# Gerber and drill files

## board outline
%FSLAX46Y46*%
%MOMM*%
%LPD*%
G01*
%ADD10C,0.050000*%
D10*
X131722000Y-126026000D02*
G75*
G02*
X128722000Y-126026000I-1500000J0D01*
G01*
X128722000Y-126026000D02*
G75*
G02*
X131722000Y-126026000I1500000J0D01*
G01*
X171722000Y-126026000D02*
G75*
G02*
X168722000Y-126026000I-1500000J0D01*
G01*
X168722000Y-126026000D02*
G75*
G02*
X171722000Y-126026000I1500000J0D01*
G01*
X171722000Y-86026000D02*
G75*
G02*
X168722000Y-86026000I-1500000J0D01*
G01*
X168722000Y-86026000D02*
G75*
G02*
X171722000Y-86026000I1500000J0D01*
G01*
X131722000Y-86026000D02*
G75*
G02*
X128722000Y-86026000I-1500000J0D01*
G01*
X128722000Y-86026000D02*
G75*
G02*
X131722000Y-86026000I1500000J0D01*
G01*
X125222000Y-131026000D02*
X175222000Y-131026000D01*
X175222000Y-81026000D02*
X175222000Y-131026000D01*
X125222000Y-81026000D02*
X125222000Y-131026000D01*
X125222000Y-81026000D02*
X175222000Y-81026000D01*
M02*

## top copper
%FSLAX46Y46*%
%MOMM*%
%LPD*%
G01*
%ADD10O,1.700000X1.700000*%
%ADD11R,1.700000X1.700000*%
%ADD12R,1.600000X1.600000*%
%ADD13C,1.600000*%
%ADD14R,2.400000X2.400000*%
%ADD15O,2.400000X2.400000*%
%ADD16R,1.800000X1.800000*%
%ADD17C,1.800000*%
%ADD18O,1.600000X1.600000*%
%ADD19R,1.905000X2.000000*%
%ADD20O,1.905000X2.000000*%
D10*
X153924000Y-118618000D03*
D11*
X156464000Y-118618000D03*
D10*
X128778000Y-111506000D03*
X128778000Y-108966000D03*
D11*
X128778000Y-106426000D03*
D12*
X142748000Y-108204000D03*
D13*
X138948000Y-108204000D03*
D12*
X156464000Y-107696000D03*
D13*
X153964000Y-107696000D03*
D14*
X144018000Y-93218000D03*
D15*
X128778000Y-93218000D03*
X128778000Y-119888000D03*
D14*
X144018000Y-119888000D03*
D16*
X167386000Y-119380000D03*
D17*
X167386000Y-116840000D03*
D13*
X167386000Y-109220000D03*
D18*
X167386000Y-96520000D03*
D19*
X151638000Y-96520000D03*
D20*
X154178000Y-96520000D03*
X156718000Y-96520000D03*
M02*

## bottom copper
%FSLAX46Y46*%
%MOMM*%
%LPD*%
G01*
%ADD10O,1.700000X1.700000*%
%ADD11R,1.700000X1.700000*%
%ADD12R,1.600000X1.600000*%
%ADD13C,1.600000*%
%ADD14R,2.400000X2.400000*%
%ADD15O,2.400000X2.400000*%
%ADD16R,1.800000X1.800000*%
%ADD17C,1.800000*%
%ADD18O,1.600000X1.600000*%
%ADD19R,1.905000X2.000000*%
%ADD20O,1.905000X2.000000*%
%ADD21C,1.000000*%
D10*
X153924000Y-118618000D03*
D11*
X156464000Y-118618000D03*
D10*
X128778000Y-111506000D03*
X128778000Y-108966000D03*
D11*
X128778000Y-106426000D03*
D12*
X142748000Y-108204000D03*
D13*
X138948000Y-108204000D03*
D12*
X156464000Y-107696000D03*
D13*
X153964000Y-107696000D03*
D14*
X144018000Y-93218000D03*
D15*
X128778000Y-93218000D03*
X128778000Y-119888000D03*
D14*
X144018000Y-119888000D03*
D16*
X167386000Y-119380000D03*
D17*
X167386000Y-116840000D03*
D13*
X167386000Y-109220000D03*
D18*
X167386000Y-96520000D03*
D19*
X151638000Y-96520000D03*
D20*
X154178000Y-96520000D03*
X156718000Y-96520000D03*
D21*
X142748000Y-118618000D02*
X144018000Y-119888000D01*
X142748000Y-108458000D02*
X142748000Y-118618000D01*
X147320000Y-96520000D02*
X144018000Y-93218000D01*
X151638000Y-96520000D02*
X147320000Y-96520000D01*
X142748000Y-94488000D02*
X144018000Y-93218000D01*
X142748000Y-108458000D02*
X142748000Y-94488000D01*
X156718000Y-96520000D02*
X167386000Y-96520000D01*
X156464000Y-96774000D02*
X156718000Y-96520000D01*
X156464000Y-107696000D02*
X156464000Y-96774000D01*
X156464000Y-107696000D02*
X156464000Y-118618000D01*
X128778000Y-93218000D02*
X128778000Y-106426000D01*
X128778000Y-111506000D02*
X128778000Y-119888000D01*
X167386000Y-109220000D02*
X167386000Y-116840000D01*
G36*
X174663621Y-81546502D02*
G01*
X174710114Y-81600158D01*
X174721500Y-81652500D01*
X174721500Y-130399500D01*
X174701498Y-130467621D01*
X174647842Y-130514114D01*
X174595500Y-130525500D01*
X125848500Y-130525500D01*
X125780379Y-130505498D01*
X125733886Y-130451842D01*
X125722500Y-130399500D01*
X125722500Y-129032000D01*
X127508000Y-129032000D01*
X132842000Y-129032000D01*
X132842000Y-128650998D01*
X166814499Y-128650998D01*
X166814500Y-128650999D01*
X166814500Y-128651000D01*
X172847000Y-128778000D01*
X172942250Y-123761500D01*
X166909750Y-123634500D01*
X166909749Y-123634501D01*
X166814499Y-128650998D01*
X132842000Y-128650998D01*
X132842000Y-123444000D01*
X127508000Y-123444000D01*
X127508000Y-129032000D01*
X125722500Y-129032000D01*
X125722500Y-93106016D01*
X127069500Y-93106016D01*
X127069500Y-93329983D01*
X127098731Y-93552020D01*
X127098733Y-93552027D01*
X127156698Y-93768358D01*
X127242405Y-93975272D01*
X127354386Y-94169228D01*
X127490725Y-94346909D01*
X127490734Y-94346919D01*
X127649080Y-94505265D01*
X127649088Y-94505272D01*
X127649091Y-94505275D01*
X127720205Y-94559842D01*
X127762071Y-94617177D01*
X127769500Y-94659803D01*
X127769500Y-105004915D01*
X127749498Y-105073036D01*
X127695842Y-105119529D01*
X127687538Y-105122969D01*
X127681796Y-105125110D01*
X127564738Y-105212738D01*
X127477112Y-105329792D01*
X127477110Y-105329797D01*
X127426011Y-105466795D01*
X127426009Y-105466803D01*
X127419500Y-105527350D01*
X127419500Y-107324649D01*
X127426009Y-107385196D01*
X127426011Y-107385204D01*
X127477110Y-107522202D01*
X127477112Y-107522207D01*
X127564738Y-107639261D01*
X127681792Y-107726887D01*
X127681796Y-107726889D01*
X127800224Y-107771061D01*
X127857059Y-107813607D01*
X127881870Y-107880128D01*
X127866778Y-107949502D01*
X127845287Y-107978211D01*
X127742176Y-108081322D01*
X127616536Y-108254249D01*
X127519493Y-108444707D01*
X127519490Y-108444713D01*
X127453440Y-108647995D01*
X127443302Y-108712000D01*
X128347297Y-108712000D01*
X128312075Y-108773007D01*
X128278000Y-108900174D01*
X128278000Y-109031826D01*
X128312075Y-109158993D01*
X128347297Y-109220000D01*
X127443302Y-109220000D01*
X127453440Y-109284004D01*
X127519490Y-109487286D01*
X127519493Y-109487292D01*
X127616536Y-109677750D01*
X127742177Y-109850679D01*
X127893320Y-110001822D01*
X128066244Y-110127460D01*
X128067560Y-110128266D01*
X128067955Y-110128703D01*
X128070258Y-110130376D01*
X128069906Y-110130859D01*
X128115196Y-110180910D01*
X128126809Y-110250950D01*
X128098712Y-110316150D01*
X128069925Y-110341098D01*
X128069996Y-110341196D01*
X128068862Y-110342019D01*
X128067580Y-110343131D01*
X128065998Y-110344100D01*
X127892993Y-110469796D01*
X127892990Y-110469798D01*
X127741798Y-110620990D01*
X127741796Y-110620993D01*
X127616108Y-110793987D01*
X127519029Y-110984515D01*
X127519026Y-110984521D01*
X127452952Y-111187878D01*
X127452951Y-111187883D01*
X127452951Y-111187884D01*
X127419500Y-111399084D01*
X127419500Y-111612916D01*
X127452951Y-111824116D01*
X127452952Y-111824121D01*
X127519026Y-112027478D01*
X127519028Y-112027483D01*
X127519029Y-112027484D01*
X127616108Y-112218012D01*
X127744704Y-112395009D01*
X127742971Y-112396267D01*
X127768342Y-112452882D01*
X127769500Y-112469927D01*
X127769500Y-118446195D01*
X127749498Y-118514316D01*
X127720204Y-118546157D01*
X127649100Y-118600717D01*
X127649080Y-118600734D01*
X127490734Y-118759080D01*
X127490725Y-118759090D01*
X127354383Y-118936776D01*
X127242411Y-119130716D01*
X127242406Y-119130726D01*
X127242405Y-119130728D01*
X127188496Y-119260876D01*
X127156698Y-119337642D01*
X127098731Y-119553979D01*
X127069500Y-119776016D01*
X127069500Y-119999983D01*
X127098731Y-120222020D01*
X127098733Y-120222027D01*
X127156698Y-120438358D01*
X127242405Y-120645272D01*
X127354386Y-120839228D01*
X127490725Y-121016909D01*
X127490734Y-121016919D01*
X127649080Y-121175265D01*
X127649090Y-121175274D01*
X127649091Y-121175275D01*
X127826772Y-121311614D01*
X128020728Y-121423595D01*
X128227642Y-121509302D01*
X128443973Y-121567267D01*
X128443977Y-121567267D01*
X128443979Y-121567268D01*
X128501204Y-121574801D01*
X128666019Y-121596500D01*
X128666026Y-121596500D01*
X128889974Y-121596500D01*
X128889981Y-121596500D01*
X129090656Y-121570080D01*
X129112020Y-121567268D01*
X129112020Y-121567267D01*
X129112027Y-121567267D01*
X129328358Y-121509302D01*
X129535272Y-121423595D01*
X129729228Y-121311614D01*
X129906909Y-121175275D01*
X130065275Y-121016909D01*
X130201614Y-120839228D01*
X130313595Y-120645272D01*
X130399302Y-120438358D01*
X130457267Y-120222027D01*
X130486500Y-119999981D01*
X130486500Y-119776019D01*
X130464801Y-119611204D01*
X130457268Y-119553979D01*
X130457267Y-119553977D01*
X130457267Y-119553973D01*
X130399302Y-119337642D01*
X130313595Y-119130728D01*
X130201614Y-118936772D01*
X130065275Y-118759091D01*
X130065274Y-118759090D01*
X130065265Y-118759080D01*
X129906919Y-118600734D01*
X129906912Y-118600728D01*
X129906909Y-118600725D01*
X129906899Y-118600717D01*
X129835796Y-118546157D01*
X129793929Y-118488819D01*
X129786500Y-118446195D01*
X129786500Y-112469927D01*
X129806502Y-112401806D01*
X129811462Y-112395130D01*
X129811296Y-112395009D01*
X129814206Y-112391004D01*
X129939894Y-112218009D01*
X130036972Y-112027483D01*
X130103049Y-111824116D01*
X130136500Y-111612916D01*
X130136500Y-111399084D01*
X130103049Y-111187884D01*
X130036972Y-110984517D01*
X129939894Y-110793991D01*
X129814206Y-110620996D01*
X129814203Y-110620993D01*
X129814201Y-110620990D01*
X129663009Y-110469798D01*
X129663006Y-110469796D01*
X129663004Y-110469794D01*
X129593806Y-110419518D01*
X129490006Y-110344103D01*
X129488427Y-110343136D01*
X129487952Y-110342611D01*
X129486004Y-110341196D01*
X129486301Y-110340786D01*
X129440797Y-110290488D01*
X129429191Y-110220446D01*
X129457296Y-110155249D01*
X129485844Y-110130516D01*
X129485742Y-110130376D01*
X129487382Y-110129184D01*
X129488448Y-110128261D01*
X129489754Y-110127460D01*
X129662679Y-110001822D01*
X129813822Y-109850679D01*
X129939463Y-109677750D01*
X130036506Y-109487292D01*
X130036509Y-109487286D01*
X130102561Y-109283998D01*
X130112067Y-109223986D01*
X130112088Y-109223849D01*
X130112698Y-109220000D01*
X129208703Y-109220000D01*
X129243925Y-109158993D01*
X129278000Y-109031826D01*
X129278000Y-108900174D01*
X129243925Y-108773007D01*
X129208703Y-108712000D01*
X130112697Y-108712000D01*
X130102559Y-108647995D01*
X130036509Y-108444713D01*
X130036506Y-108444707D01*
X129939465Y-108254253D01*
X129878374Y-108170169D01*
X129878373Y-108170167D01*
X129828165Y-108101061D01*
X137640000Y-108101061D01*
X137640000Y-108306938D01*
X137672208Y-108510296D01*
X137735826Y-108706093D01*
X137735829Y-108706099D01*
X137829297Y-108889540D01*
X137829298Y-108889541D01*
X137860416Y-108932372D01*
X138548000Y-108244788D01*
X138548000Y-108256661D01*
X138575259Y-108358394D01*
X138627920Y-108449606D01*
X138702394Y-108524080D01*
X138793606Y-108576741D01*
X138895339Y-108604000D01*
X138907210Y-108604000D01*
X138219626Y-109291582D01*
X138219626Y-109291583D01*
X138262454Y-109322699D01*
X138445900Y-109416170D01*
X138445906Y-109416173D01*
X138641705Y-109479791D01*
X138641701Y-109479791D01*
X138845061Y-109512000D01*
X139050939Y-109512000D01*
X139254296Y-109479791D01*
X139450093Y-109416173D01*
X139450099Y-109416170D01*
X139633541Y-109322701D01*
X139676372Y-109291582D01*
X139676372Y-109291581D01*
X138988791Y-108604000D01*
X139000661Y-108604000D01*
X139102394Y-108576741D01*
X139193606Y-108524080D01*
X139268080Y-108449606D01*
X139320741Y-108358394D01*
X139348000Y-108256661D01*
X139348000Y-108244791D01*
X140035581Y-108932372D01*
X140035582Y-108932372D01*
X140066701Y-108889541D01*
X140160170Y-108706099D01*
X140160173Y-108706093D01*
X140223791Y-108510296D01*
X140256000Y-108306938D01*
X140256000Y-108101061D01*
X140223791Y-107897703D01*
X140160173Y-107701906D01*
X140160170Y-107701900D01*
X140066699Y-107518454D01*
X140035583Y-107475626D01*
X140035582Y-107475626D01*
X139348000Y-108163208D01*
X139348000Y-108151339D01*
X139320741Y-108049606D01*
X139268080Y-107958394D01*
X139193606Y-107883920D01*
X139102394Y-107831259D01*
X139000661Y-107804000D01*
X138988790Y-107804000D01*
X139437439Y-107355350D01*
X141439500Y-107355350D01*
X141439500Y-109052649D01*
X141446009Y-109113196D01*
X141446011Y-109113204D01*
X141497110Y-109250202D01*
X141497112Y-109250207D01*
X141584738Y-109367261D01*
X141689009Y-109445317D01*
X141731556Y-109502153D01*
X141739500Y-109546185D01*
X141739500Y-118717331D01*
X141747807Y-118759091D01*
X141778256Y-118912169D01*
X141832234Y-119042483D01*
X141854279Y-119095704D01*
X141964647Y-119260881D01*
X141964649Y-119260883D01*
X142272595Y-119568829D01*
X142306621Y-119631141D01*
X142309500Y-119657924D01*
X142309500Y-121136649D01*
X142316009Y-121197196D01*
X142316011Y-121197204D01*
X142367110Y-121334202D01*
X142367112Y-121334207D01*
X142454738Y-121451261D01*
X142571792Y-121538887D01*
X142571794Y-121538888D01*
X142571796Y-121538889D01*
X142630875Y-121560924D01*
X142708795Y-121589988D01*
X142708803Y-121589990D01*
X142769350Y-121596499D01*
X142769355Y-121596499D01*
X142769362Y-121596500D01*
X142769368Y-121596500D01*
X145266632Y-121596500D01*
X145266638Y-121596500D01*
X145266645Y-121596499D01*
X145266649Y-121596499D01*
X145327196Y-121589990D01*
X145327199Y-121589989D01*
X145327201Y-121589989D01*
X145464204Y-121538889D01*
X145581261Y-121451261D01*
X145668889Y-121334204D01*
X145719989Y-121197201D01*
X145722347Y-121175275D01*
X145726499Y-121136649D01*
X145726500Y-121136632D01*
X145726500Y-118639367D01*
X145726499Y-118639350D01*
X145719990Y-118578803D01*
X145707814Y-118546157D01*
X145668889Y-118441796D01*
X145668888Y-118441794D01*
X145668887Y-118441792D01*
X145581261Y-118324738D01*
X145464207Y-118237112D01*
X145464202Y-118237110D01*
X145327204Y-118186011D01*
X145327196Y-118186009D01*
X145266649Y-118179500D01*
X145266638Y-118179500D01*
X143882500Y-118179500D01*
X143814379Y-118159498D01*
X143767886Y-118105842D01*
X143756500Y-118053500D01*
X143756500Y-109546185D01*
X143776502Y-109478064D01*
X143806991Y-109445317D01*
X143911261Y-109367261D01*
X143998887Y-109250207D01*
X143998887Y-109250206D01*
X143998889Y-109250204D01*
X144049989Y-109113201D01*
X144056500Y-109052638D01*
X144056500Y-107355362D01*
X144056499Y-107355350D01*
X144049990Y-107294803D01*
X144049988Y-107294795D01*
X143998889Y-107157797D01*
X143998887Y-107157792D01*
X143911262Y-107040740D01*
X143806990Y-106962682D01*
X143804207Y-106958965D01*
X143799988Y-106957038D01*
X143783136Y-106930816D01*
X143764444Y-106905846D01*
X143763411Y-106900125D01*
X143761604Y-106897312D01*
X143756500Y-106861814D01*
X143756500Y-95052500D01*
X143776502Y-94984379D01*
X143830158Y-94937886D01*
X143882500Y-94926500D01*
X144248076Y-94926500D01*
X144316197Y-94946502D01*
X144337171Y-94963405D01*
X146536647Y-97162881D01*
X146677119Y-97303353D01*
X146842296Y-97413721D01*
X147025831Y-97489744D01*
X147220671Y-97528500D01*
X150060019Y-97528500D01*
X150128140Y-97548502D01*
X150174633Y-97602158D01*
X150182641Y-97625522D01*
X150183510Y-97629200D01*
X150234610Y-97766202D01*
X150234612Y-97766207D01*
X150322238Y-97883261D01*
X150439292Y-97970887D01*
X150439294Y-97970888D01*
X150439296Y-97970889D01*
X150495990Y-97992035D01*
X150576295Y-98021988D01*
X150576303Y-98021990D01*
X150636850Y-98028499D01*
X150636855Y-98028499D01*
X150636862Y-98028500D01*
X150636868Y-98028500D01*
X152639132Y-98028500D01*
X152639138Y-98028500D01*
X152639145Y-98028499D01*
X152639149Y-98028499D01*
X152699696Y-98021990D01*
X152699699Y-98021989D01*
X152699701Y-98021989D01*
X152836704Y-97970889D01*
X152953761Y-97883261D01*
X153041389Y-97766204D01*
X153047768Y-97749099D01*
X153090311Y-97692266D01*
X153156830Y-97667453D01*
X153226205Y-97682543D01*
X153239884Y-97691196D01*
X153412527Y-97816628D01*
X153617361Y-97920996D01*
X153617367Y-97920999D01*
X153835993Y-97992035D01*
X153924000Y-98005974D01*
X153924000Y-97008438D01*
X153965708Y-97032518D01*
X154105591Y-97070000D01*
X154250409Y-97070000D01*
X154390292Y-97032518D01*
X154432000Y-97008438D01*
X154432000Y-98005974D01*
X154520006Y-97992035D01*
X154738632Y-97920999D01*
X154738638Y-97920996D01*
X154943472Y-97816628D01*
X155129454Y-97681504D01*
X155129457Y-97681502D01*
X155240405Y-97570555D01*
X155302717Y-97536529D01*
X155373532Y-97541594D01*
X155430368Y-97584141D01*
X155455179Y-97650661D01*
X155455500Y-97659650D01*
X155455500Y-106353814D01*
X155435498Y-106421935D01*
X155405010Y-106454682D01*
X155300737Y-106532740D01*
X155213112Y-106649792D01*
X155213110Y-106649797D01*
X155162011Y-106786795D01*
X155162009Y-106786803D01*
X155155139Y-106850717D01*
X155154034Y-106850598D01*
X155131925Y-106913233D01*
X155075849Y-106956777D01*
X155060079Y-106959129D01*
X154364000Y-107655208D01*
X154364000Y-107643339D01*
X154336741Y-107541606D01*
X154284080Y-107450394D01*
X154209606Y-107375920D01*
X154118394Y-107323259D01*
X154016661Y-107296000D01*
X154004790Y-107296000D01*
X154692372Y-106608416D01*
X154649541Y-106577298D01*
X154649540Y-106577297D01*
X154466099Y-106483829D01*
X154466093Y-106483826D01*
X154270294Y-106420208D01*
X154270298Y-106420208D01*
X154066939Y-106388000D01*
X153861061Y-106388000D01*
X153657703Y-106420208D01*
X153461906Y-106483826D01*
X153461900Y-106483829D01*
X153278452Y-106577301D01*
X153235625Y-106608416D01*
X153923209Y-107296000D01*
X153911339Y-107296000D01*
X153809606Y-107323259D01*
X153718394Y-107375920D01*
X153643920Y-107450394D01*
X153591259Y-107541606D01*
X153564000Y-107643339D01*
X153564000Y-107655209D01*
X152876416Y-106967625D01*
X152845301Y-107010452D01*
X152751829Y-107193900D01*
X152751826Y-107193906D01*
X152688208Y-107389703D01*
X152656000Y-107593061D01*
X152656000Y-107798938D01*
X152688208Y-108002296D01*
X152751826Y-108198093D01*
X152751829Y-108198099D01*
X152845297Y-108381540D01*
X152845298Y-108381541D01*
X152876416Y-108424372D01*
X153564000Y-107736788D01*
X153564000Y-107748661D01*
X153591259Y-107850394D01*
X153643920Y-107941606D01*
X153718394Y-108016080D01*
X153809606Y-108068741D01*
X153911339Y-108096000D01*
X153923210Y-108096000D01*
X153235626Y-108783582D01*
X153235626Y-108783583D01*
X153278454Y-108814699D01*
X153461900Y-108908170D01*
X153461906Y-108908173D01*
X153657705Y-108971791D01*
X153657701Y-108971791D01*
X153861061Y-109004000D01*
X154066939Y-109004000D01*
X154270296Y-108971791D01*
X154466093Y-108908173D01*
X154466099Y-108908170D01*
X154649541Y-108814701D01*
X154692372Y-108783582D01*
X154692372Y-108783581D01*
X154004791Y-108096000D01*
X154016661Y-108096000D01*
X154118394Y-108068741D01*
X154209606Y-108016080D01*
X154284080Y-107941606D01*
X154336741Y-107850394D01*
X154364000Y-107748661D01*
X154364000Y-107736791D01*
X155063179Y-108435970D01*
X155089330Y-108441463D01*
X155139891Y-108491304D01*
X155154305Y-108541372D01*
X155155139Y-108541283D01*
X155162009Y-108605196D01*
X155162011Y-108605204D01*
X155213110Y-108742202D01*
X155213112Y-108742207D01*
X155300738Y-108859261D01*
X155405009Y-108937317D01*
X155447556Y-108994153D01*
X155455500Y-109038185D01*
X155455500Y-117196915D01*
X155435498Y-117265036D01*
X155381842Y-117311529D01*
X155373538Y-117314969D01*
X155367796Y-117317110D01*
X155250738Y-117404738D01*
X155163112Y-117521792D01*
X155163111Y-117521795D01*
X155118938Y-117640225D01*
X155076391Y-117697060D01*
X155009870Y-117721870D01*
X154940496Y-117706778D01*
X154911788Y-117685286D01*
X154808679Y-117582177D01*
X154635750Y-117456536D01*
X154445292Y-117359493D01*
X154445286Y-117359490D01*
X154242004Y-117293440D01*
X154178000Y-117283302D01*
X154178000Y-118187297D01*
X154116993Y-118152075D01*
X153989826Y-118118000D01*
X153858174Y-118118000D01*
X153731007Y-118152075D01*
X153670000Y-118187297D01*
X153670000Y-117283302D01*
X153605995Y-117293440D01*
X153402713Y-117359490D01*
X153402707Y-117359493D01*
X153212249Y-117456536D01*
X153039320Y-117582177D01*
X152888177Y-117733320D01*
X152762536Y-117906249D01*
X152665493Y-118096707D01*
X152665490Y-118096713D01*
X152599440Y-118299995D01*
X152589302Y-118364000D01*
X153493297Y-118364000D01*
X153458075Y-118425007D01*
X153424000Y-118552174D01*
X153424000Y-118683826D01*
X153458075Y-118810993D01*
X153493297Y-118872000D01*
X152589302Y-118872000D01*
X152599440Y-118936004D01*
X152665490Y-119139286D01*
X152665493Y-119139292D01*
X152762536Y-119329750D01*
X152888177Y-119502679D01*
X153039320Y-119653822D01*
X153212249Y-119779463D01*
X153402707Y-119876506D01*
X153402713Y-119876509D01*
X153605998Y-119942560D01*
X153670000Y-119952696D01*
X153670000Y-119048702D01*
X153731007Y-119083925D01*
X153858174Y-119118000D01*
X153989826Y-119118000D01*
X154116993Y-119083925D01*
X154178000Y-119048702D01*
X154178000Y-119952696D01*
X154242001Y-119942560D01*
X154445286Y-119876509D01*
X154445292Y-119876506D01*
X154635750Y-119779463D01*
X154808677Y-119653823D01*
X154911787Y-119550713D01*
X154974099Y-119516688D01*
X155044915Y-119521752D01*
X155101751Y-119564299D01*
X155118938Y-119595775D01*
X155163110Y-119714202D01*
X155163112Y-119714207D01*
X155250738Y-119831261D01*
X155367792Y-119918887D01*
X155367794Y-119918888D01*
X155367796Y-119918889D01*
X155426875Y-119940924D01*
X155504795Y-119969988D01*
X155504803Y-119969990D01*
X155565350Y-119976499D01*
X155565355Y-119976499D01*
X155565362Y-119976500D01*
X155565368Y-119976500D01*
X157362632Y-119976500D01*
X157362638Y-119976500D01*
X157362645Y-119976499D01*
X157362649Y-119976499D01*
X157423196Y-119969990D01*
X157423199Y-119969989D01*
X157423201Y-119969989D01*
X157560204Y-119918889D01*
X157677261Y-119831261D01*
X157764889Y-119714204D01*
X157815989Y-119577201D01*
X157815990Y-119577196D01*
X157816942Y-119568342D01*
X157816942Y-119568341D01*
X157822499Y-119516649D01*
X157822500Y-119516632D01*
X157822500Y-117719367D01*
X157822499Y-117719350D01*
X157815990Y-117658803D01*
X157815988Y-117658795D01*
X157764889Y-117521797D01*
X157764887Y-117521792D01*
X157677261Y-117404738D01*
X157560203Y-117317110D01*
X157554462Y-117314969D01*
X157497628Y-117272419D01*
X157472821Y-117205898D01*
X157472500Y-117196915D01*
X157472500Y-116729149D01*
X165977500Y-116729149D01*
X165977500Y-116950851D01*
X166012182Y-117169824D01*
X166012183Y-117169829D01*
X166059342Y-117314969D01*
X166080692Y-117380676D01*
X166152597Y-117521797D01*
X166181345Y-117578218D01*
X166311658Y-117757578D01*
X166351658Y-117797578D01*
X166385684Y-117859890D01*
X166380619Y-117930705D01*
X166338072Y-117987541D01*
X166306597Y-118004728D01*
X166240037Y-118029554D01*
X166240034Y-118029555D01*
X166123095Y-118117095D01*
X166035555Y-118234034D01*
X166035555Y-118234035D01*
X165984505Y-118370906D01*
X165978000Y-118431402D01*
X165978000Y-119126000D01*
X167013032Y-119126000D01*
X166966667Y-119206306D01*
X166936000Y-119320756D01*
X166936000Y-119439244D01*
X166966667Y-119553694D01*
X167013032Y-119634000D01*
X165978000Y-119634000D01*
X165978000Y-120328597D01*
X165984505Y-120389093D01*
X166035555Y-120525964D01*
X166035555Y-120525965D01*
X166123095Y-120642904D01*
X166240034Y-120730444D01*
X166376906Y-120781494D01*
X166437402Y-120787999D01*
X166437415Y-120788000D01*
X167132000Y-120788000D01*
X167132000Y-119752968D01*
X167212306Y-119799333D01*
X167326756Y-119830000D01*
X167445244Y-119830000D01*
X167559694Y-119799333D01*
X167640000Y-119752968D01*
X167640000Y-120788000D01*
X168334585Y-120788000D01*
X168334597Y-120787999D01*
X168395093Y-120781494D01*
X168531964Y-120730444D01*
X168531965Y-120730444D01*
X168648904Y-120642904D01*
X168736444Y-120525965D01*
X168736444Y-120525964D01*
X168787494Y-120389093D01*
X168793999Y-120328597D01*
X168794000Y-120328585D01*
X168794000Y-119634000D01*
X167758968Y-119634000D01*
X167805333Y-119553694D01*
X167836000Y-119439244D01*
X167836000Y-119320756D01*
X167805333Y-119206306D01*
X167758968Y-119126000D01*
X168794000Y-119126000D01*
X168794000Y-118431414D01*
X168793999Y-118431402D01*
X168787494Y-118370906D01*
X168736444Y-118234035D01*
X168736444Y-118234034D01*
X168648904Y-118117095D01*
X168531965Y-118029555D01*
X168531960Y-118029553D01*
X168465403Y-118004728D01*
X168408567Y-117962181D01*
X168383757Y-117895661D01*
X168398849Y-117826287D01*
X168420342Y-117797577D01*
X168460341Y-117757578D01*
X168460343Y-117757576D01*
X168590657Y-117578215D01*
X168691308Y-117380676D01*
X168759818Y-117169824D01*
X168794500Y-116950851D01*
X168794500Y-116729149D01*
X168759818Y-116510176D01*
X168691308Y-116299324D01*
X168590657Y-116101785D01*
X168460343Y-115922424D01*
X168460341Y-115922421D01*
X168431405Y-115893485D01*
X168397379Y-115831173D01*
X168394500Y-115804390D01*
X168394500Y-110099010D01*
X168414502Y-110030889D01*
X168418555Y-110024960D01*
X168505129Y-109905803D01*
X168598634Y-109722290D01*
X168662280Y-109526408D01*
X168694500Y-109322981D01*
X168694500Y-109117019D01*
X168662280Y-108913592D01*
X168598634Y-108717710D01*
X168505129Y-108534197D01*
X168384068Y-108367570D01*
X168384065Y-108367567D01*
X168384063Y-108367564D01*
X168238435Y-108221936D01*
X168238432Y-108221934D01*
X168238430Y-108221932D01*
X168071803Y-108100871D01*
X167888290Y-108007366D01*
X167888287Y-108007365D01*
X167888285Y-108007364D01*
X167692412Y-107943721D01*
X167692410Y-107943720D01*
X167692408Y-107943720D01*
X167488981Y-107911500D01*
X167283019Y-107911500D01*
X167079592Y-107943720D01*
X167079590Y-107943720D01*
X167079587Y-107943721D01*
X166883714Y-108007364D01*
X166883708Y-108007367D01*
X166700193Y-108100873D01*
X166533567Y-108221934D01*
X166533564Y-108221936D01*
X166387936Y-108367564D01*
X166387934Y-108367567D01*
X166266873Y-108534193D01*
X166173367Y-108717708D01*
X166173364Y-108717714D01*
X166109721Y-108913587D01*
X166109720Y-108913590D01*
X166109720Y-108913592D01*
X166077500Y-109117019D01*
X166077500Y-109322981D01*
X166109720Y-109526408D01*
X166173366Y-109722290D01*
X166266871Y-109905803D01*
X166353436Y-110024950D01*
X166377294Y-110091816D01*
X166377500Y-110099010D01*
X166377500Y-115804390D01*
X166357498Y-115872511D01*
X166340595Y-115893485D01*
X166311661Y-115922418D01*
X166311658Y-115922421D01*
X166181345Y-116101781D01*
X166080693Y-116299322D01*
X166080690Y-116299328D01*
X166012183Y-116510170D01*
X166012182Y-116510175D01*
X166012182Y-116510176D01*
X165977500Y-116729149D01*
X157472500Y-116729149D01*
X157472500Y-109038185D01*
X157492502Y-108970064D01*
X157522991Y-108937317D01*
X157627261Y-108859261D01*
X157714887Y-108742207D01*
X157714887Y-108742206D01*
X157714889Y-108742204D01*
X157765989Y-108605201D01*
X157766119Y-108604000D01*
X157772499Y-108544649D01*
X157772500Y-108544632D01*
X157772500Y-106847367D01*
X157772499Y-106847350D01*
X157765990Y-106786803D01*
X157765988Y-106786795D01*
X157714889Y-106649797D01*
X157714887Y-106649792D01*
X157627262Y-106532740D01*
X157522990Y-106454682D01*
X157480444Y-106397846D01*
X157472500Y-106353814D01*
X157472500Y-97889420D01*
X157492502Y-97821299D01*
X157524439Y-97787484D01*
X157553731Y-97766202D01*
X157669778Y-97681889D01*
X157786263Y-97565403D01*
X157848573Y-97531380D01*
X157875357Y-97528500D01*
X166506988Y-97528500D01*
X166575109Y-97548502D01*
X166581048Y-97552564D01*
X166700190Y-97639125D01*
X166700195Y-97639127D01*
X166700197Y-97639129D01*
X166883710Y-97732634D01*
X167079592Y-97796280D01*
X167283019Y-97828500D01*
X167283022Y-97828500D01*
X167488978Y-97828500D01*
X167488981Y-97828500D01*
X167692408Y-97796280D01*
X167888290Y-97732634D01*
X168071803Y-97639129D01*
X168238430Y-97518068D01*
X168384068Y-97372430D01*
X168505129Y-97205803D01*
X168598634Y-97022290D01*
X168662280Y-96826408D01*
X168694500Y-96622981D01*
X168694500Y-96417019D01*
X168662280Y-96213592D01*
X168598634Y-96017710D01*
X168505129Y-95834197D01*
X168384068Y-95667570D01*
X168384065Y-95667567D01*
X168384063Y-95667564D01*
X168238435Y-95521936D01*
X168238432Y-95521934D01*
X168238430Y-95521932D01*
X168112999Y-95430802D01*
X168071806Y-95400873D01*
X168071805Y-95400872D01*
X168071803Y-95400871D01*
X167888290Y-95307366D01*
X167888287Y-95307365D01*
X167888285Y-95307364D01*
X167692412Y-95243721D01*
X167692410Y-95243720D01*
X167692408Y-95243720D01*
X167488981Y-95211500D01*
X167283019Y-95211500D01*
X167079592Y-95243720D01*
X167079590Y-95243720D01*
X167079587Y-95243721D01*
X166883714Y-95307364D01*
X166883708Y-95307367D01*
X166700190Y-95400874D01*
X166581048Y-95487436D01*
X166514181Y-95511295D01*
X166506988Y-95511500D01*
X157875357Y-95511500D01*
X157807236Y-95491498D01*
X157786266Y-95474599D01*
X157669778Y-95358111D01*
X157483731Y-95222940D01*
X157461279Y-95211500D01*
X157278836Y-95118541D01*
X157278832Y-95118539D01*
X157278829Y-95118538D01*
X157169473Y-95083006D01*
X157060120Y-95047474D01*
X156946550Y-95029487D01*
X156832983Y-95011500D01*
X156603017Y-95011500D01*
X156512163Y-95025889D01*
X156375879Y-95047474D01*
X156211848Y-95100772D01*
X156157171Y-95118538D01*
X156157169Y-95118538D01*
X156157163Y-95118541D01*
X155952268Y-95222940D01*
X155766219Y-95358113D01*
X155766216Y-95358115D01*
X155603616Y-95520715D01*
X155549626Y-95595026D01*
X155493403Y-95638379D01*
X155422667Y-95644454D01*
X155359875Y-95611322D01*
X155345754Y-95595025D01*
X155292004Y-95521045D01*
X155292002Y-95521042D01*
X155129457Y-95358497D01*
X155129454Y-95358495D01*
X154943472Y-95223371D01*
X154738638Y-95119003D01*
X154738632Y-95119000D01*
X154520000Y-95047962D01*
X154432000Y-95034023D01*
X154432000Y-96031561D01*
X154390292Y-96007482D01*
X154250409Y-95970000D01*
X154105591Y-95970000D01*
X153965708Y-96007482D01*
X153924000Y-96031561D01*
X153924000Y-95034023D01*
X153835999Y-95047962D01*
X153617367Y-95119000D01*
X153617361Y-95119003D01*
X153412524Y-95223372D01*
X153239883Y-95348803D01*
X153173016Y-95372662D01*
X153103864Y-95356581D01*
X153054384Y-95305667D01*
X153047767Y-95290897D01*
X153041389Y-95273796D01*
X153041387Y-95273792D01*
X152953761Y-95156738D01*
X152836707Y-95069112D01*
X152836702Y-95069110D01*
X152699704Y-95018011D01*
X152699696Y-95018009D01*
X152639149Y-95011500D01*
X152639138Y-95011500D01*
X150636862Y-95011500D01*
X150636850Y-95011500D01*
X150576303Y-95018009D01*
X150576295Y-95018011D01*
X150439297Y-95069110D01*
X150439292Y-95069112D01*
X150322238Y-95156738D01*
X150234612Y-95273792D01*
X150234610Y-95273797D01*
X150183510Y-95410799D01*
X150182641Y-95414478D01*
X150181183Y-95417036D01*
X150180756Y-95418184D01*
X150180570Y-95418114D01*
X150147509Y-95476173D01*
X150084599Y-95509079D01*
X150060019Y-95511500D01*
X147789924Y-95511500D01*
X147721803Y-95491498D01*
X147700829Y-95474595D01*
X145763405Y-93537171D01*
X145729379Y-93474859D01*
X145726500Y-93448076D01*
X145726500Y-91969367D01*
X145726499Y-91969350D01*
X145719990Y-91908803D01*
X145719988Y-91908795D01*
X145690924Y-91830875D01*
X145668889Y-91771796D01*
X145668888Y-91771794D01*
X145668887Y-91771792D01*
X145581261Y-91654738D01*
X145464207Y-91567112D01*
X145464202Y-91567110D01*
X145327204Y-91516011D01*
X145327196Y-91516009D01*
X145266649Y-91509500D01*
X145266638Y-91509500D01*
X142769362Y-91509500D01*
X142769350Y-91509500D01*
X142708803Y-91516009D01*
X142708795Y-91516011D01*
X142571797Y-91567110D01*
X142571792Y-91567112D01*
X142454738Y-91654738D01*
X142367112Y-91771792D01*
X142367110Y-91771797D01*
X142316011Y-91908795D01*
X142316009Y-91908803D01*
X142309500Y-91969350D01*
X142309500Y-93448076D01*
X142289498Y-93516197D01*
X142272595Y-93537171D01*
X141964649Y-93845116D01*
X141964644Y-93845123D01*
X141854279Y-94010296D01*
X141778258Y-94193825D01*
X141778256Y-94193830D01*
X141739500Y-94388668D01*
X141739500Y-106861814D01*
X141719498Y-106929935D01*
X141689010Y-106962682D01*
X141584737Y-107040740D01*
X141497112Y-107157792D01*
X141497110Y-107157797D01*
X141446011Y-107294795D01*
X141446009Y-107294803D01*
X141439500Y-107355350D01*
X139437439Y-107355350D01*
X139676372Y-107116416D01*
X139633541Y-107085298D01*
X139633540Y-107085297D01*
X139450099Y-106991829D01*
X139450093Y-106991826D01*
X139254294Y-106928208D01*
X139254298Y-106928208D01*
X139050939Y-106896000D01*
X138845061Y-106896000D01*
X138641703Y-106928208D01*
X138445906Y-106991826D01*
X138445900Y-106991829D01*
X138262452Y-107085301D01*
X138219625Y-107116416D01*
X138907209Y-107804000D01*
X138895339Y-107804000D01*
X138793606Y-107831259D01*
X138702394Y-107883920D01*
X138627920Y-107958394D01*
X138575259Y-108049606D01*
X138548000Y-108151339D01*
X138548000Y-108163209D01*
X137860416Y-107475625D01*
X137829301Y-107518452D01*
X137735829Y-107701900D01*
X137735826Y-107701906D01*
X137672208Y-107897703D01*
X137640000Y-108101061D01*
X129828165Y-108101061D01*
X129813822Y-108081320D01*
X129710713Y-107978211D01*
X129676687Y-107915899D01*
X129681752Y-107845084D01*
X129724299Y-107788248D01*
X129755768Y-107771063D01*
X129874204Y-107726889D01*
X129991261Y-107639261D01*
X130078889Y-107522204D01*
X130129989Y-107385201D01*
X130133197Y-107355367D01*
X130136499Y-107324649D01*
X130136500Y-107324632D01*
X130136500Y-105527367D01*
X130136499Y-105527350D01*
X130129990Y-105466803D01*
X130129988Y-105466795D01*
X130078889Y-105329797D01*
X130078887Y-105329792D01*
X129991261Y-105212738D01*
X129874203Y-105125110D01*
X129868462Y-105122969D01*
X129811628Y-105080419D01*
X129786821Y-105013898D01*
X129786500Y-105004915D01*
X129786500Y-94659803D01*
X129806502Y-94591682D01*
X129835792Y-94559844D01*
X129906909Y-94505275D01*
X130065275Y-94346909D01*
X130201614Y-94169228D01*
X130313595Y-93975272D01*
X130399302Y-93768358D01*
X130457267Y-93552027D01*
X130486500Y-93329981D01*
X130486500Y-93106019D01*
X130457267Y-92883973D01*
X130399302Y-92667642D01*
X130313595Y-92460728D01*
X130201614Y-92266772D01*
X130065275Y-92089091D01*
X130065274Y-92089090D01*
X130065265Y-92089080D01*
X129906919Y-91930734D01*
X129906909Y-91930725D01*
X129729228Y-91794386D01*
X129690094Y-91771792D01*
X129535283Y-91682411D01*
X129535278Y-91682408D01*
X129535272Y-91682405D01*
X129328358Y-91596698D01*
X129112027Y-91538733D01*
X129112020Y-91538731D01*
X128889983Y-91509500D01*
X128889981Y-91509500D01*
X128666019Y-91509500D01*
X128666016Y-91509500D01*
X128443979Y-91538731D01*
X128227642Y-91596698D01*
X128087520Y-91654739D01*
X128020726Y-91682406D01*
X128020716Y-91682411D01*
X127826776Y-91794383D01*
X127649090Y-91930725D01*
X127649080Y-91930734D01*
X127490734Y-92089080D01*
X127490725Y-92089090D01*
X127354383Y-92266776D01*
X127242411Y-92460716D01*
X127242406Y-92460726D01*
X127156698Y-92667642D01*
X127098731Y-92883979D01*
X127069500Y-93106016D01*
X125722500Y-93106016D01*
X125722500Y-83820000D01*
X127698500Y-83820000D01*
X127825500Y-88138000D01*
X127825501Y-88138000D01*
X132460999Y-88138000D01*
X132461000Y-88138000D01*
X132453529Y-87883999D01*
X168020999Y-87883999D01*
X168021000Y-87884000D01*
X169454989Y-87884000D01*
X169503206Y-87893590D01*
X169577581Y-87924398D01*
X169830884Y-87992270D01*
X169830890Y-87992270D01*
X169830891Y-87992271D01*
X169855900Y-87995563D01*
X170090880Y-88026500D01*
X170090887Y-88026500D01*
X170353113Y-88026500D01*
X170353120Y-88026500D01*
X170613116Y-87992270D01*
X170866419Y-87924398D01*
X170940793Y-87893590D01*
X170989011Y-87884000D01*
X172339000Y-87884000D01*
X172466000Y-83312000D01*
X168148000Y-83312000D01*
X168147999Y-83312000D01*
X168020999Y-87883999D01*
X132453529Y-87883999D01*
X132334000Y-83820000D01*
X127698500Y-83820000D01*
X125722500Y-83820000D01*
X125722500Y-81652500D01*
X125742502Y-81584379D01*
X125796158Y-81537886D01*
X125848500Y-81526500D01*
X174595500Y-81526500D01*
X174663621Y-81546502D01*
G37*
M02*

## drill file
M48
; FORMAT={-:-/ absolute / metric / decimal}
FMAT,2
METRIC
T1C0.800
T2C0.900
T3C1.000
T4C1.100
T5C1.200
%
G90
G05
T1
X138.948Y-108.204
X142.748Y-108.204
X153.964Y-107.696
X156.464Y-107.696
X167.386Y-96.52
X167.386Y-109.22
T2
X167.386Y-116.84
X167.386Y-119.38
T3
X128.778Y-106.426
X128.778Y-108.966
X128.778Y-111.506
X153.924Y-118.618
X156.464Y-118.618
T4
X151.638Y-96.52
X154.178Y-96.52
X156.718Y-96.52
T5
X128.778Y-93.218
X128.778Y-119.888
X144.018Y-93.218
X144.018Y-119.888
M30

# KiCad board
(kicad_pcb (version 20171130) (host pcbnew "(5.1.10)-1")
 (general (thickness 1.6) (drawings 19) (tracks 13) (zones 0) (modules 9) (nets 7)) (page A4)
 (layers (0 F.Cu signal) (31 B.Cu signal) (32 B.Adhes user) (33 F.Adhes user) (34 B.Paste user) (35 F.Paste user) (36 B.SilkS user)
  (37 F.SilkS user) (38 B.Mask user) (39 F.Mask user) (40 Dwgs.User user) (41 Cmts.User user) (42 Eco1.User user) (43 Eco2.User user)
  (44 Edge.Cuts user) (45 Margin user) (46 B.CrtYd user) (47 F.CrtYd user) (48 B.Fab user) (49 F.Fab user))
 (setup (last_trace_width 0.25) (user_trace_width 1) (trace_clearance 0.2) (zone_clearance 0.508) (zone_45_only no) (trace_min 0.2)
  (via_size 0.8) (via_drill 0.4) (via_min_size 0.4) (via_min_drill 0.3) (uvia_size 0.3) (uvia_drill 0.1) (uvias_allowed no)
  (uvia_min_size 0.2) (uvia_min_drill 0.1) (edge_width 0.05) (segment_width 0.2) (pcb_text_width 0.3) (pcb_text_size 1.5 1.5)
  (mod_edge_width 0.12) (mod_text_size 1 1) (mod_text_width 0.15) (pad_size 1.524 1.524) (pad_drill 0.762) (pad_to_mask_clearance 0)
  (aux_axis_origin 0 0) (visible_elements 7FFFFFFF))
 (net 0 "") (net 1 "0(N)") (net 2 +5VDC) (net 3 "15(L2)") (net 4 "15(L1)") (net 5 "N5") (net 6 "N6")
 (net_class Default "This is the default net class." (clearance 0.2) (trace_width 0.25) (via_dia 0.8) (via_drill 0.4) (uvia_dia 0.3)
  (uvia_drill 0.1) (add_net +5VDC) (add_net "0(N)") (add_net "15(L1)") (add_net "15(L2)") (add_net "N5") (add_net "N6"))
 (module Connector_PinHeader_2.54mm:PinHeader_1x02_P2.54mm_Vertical (layer F.Cu) (at 156.464 118.618 270)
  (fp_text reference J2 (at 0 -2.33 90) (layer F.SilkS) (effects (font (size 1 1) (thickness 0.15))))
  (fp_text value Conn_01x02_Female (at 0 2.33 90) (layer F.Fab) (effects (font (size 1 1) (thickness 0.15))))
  (pad 2 thru_hole oval (at 0 2.54 270) (size 1.7 1.7) (drill 1) (layers *.Cu *.Mask) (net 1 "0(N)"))
  (pad 1 thru_hole rect (at 0 0 270) (size 1.7 1.7) (drill 1) (layers *.Cu *.Mask) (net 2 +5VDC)))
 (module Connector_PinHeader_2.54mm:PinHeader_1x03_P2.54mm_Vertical (layer F.Cu) (at 128.778 106.426)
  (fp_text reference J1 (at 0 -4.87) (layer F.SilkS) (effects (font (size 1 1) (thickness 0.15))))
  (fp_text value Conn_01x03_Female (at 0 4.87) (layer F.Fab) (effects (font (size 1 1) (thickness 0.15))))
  (pad 3 thru_hole oval (at 0 5.08) (size 1.7 1.7) (drill 1) (layers *.Cu *.Mask) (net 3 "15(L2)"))
  (pad 2 thru_hole oval (at 0 2.54) (size 1.7 1.7) (drill 1) (layers *.Cu *.Mask) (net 1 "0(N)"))
  (pad 1 thru_hole rect (at 0 0) (size 1.7 1.7) (drill 1) (layers *.Cu *.Mask) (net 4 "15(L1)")))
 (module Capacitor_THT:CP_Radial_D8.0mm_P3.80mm (layer F.Cu) (at 142.748 108.204 180)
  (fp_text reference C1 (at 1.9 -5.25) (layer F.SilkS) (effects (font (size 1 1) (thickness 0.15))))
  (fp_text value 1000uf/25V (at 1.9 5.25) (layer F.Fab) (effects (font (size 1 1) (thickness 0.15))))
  (pad 1 thru_hole rect (at 0 0 180) (size 1.6 1.6) (drill 0.8) (layers *.Cu *.Mask) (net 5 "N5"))
  (pad 2 thru_hole circle (at 3.8 0 180) (size 1.6 1.6) (drill 0.8) (layers *.Cu *.Mask) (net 1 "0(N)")))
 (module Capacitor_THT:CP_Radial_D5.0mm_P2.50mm (layer F.Cu) (at 156.464 107.696 180)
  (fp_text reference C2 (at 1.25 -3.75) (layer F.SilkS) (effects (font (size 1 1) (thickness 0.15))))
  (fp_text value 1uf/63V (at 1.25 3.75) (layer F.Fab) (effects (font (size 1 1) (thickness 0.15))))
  (pad 1 thru_hole rect (at 0 0 180) (size 1.6 1.6) (drill 0.8) (layers *.Cu *.Mask) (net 2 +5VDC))
  (pad 2 thru_hole circle (at 2.5 0 180) (size 1.6 1.6) (drill 0.8) (layers *.Cu *.Mask) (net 1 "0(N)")))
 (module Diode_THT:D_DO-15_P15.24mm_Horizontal (layer F.Cu) (at 144.018 93.218 180)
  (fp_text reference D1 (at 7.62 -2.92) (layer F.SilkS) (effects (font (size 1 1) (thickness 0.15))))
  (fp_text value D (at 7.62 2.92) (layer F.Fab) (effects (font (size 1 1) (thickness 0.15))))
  (pad 1 thru_hole rect (at 0 0 180) (size 2.4 2.4) (drill 1.2) (layers *.Cu *.Mask) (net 5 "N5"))
  (pad 2 thru_hole oval (at 15.24 0 180) (size 2.4 2.4) (drill 1.2) (layers *.Cu *.Mask) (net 4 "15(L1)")))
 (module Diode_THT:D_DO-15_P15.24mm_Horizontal (layer F.Cu) (at 144.018 119.888 180)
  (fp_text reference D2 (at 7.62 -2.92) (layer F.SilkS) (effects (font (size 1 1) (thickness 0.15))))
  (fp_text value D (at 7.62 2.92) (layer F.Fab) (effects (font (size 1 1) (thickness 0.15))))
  (pad 2 thru_hole oval (at 15.24 0 180) (size 2.4 2.4) (drill 1.2) (layers *.Cu *.Mask) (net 3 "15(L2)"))
  (pad 1 thru_hole rect (at 0 0 180) (size 2.4 2.4) (drill 1.2) (layers *.Cu *.Mask) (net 5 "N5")))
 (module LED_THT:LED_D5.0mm (layer F.Cu) (at 167.386 119.38 90)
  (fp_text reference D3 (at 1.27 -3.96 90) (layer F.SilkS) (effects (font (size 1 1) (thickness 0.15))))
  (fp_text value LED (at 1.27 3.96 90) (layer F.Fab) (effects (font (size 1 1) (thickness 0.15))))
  (pad 1 thru_hole rect (at 0 0 90) (size 1.8 1.8) (drill 0.9) (layers *.Cu *.Mask) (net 1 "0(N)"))
  (pad 2 thru_hole circle (at 2.54 0 90) (size 1.8 1.8) (drill 0.9) (layers *.Cu *.Mask) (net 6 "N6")))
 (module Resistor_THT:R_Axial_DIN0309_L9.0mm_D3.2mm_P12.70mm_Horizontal (layer F.Cu) (at 167.386 109.22 90)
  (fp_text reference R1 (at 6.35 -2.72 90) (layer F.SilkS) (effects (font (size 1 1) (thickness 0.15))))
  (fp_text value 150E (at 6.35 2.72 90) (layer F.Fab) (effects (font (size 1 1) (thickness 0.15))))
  (pad 1 thru_hole circle (at 0 0 90) (size 1.6 1.6) (drill 0.8) (layers *.Cu *.Mask) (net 6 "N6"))
  (pad 2 thru_hole oval (at 12.7 0 90) (size 1.6 1.6) (drill 0.8) (layers *.Cu *.Mask) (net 2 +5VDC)))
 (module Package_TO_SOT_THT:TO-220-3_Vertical (layer F.Cu) (at 151.638 96.52)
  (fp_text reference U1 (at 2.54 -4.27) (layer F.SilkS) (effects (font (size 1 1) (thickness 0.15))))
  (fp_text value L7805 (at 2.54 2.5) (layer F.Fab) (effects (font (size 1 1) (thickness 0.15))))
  (pad 1 thru_hole rect (at 0 0) (size 1.905 2) (drill 1.1) (layers *.Cu *.Mask) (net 5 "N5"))
  (pad 2 thru_hole oval (at 2.54 0) (size 1.905 2) (drill 1.1) (layers *.Cu *.Mask) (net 1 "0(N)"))
  (pad 3 thru_hole oval (at 5.08 0) (size 1.905 2) (drill 1.1) (layers *.Cu *.Mask) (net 2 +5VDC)))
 (gr_circle (center 130.222 126.026) (end 131.722 126.026) (layer Edge.Cuts) (width 0.05))
 (gr_circle (center 170.222 126.026) (end 171.722 126.026) (layer Edge.Cuts) (width 0.05))
 (gr_circle (center 170.222 86.026) (end 171.722 86.026) (layer Edge.Cuts) (width 0.05))
 (gr_circle (center 130.222 86.026) (end 131.722 86.026) (layer Edge.Cuts) (width 0.05))
 (gr_line (start 125.222 131.026) (end 175.222 131.026) (layer Edge.Cuts) (width 0.05))
 (gr_line (start 175.222 81.026) (end 175.222 131.026) (layer Edge.Cuts) (width 0.05))
 (gr_line (start 125.222 81.026) (end 125.222 131.026) (layer Edge.Cuts) (width 0.05))
 (gr_line (start 125.222 81.026) (end 175.222 81.026) (layer Edge.Cuts) (width 0.05))
 (segment (start 142.748 118.618) (end 144.018 119.888) (width 1) (layer B.Cu) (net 5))
 (segment (start 142.748 108.458) (end 142.748 118.618) (width 1) (layer B.Cu) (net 5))
 (segment (start 147.32 96.52) (end 144.018 93.218) (width 1) (layer B.Cu) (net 5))
 (segment (start 151.638 96.52) (end 147.32 96.52) (width 1) (layer B.Cu) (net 5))
 (segment (start 142.748 94.488) (end 144.018 93.218) (width 1) (layer B.Cu) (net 5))
 (segment (start 142.748 108.458) (end 142.748 94.488) (width 1) (layer B.Cu) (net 5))
 (segment (start 156.718 96.52) (end 167.386 96.52) (width 1) (layer B.Cu) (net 2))
 (segment (start 156.464 96.774) (end 156.718 96.52) (width 1) (layer B.Cu) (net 2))
 (segment (start 156.464 107.696) (end 156.464 96.774) (width 1) (layer B.Cu) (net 2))
 (segment (start 156.464 107.696) (end 156.464 118.618) (width 1) (layer B.Cu) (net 2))
 (segment (start 128.778 93.218) (end 128.778 106.426) (width 1) (layer B.Cu) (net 4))
 (segment (start 128.778 111.506) (end 128.778 119.888) (width 1) (layer B.Cu) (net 3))
 (segment (start 167.386 109.22) (end 167.386 116.84) (width 1) (layer B.Cu) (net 6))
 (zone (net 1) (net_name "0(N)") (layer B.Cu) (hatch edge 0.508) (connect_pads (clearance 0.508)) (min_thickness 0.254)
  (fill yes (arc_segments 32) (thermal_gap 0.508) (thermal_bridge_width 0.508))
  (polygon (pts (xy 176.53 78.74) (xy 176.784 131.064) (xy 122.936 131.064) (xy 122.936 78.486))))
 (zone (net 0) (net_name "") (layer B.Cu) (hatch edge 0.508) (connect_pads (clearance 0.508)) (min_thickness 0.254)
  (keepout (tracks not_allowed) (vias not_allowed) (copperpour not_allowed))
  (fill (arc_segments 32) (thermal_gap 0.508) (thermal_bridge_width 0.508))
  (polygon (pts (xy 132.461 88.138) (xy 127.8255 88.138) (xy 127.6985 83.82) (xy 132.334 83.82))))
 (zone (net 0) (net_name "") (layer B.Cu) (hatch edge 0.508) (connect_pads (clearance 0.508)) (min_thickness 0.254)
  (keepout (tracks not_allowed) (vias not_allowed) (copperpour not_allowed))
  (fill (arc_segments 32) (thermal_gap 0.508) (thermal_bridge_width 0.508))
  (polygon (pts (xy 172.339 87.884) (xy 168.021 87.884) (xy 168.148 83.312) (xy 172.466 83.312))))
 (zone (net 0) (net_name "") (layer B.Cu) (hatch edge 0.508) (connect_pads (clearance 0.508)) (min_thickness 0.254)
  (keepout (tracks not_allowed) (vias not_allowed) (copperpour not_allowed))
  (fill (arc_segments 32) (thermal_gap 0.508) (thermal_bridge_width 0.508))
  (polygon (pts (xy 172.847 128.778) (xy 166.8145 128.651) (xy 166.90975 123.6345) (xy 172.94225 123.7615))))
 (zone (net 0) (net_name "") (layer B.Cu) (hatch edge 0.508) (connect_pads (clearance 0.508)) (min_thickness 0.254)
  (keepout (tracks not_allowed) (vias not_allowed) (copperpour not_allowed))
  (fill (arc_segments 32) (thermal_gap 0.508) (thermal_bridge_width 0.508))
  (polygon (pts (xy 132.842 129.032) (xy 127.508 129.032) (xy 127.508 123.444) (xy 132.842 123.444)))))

